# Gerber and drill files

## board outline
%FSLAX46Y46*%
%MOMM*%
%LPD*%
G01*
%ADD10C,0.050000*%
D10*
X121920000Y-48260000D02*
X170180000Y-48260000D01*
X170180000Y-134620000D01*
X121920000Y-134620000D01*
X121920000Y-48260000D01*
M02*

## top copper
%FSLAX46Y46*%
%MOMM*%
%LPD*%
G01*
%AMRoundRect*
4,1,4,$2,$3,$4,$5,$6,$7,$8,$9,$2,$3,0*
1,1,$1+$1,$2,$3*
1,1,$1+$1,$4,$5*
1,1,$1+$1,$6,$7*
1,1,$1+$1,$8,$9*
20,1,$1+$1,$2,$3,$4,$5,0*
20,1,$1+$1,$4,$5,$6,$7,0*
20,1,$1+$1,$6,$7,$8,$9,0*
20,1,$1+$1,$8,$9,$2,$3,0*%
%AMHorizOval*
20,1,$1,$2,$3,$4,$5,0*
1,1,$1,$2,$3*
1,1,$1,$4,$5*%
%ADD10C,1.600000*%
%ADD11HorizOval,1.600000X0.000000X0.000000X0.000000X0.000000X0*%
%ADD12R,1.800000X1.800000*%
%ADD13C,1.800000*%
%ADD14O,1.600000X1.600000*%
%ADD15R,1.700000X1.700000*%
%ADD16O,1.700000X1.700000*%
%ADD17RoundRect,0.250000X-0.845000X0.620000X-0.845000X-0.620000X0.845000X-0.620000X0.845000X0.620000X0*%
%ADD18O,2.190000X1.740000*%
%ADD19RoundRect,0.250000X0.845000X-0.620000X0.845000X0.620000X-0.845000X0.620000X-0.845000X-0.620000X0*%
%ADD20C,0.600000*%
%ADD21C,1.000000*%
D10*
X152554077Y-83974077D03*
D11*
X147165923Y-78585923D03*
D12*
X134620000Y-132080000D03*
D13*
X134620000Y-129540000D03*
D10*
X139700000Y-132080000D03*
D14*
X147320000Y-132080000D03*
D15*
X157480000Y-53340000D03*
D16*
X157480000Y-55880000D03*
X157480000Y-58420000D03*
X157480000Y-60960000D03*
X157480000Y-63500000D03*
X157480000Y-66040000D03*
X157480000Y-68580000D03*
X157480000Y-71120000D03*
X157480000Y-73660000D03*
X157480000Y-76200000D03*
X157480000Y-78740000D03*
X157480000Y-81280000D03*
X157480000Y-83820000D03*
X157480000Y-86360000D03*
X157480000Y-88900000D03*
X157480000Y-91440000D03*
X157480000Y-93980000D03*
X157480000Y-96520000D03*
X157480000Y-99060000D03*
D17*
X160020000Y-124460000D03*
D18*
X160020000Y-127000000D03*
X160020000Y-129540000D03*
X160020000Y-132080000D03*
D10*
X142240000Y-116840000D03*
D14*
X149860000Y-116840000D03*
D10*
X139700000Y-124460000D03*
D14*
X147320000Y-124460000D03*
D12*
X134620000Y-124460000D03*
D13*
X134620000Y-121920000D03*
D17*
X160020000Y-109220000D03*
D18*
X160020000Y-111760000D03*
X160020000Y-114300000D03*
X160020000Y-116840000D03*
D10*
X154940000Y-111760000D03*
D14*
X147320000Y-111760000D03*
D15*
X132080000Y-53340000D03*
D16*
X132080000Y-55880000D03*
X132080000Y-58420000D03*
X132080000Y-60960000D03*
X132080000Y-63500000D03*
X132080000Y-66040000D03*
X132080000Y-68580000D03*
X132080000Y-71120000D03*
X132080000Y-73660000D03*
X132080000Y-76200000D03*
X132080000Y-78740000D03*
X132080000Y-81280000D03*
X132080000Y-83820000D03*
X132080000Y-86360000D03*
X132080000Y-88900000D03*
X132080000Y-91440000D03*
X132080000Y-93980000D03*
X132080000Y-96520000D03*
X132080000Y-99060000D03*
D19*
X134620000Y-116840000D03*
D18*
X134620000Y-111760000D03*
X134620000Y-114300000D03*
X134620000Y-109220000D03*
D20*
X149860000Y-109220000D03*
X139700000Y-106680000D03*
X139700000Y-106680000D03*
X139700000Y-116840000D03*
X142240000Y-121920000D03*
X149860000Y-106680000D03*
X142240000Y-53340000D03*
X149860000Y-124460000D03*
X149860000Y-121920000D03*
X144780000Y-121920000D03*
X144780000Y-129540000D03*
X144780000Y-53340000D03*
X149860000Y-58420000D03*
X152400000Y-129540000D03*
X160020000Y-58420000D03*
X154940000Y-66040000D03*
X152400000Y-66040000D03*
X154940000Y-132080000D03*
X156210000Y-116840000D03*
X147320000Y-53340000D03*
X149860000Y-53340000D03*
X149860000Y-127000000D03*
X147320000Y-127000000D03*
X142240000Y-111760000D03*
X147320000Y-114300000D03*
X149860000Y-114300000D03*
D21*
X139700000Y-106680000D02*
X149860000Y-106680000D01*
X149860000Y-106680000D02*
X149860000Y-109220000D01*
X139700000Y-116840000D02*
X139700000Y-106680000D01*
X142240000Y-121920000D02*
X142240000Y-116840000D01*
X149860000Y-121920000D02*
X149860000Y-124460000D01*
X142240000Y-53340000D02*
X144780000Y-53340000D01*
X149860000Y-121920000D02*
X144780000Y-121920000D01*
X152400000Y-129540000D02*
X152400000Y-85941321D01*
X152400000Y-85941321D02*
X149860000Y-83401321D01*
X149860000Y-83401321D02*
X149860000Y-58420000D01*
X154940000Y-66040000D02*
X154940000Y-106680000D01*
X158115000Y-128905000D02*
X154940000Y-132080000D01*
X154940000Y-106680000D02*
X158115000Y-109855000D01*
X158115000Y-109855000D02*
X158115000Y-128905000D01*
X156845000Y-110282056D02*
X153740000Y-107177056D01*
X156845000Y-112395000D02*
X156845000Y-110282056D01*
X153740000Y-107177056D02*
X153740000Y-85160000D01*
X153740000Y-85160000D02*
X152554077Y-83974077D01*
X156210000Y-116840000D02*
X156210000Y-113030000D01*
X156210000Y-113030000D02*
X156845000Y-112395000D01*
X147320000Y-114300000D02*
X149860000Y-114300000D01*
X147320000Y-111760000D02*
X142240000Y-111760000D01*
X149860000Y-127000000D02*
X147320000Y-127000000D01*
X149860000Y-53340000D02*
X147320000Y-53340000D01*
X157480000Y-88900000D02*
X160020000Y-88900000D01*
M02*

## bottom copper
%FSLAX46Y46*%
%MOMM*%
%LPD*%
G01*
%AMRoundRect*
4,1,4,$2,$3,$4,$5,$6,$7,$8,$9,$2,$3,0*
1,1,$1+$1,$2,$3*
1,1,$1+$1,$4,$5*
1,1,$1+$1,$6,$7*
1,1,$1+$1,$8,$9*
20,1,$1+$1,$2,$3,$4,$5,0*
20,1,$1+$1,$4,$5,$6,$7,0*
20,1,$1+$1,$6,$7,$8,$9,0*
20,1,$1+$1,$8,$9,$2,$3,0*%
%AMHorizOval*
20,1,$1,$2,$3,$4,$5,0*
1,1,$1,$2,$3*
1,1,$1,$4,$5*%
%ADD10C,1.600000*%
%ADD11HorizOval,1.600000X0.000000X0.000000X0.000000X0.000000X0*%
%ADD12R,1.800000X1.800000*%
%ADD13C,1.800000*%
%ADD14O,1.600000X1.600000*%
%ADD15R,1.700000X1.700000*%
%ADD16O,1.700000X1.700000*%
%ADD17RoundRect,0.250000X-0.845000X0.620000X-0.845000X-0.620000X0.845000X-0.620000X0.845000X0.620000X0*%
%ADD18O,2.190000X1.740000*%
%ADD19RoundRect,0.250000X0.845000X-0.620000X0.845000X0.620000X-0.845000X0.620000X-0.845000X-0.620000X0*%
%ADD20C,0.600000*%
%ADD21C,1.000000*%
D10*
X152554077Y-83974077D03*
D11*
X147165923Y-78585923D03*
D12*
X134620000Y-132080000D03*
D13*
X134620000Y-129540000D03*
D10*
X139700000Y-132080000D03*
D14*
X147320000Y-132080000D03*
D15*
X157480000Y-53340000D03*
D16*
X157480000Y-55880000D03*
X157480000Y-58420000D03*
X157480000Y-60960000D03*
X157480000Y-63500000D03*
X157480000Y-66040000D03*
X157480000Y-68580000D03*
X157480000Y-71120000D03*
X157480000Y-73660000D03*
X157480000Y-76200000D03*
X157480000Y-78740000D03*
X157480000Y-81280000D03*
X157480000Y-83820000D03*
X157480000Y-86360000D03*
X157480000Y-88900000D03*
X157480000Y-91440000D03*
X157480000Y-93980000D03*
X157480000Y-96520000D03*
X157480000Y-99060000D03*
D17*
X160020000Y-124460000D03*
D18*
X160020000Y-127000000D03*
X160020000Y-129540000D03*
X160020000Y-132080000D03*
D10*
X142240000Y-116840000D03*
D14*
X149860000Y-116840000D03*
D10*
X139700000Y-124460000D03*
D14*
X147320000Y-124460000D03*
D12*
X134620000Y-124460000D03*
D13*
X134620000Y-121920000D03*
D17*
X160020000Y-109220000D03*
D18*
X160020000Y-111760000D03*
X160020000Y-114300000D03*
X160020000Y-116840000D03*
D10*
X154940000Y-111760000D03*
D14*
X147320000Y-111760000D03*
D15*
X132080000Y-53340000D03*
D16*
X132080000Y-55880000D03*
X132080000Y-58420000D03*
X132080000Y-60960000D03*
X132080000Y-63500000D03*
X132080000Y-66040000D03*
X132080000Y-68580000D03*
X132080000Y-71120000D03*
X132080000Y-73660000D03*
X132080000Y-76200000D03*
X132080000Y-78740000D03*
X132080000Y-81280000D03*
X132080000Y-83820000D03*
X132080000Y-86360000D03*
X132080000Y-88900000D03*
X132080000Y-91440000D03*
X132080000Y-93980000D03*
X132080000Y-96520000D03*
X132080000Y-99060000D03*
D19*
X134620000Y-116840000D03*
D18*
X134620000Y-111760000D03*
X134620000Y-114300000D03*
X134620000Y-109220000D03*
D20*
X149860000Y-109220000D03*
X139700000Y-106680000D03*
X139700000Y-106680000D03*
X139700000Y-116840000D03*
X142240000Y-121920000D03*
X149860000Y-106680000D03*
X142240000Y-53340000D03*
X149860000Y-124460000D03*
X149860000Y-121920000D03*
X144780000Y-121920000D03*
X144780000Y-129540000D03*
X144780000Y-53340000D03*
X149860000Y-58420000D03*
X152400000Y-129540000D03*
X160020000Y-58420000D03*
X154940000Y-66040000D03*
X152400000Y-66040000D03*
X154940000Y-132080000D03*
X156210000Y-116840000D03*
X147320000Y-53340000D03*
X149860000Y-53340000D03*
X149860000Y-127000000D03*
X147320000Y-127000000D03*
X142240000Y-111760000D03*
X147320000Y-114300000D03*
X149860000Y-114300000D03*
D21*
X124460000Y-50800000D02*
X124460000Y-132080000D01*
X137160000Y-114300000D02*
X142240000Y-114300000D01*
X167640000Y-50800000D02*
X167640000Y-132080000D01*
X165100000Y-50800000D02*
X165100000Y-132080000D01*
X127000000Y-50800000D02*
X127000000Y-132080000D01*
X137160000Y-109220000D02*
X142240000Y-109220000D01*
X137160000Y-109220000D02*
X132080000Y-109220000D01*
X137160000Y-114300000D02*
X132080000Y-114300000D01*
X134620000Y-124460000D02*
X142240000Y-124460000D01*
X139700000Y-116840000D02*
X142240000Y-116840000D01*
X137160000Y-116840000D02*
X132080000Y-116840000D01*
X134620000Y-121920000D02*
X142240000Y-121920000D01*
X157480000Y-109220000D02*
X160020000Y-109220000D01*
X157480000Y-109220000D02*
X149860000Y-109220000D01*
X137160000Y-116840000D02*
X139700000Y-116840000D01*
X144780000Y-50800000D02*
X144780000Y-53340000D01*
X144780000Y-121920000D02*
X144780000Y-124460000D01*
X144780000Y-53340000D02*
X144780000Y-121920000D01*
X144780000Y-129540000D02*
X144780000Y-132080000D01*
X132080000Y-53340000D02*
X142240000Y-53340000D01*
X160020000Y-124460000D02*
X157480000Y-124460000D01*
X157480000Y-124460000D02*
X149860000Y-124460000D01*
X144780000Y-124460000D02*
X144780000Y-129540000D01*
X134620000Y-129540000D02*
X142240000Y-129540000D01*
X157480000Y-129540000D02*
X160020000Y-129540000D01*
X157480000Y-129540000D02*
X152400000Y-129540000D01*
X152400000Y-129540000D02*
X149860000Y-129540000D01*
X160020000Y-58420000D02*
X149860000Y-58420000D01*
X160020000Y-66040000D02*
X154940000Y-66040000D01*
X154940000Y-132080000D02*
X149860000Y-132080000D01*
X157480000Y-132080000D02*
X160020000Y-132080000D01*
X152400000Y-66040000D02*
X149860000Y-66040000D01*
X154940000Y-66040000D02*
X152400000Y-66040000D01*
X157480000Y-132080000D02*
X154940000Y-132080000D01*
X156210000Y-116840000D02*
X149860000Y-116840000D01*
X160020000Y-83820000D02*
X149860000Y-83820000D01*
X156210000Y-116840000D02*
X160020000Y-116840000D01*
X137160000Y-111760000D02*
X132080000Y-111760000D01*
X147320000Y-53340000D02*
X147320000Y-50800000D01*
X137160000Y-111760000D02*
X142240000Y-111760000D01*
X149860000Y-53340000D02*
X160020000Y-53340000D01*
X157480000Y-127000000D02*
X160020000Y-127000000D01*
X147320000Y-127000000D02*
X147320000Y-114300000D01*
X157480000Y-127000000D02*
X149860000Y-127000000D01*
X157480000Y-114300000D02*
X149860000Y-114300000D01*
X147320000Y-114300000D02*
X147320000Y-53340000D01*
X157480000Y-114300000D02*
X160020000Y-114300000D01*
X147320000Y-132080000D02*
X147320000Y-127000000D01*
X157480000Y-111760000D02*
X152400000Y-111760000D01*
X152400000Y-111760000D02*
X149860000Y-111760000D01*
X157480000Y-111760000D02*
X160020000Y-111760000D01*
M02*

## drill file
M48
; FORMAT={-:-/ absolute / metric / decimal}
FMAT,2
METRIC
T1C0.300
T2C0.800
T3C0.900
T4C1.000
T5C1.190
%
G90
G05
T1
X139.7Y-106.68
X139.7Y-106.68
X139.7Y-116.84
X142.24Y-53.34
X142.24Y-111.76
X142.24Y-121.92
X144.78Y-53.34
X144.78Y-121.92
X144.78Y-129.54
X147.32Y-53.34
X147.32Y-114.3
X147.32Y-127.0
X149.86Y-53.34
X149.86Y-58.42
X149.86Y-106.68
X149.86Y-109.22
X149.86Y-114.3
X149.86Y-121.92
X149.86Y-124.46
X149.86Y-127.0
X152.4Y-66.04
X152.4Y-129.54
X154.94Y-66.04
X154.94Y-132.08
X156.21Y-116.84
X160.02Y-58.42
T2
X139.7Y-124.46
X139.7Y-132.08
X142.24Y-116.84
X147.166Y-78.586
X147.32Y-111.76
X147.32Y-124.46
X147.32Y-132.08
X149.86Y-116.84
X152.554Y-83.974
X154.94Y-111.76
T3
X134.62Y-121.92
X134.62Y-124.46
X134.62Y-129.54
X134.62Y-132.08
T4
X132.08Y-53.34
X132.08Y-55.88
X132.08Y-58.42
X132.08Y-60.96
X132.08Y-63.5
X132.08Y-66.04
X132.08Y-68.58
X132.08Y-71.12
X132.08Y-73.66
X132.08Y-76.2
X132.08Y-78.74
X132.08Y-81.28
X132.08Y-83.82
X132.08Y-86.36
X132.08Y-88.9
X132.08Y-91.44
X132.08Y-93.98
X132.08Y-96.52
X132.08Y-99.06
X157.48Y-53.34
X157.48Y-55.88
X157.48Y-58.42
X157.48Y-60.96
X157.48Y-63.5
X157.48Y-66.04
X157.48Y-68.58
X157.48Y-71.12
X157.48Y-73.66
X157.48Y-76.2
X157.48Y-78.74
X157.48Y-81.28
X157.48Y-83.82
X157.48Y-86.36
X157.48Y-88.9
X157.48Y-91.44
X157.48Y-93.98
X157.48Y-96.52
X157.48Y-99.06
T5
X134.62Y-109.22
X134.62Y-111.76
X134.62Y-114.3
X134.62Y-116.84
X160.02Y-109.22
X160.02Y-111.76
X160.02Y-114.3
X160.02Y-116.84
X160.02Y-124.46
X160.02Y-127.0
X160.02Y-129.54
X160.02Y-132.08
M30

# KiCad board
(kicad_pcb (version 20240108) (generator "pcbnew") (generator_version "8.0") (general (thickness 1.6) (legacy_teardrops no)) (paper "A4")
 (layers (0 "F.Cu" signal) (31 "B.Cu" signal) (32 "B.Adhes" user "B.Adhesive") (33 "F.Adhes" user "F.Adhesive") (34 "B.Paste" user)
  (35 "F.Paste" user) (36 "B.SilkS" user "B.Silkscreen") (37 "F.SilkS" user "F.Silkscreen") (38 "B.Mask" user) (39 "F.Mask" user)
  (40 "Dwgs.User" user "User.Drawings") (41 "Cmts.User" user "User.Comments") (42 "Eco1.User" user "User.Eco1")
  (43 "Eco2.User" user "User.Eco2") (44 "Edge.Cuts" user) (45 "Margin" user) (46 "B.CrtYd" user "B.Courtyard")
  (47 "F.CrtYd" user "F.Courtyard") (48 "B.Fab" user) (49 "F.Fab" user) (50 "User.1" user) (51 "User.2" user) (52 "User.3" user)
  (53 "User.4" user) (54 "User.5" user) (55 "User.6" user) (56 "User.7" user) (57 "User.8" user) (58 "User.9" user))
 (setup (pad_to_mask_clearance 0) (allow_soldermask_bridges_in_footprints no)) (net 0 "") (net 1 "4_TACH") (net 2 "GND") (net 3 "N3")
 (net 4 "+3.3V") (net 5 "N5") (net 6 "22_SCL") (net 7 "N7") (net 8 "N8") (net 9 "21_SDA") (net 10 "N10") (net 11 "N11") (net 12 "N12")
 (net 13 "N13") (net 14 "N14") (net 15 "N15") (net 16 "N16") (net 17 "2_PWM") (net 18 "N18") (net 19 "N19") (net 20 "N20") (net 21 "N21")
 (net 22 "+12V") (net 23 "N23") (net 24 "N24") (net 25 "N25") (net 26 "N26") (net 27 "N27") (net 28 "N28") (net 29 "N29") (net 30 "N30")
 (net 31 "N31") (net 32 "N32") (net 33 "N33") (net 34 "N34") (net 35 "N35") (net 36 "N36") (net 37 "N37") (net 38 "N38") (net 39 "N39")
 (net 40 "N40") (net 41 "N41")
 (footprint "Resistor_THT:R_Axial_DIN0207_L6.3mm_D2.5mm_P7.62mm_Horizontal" (layer "F.Cu") (at 152.554077 83.974077 135)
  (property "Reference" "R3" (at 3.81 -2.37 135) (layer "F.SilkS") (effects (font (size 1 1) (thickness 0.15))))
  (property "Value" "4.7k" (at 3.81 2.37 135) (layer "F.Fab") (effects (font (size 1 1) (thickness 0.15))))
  (pad "1" thru_hole circle (at 0 0 135) (size 1.6 1.6) (drill 0.8) (layers "*.Cu" "*.Mask") (remove_unused_layers no) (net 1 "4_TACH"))
  (pad "2" thru_hole oval (at 7.62 0 135) (size 1.6 1.6) (drill 0.8) (layers "*.Cu" "*.Mask") (remove_unused_layers no) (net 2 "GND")))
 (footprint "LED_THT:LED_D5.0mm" (layer "F.Cu") (at 134.62 132.08 90)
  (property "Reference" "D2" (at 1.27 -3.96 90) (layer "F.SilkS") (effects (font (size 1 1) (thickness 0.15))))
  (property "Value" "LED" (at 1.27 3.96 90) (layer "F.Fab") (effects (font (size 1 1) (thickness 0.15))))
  (pad "1" thru_hole rect (at 0 0 90) (size 1.8 1.8) (drill 0.9) (layers "*.Cu" "*.Mask") (remove_unused_layers no) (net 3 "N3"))
  (pad "2" thru_hole circle (at 2.54 0 90) (size 1.8 1.8) (drill 0.9) (layers "*.Cu" "*.Mask") (remove_unused_layers no) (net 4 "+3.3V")))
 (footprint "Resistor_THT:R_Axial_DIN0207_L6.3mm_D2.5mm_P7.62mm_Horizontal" (layer "F.Cu") (at 139.7 132.08)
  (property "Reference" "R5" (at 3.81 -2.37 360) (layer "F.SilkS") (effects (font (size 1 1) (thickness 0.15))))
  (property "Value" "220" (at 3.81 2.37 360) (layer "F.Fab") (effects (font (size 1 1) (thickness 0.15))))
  (pad "1" thru_hole circle (at 0 0) (size 1.6 1.6) (drill 0.8) (layers "*.Cu" "*.Mask") (remove_unused_layers no) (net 3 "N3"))
  (pad "2" thru_hole oval (at 7.62 0) (size 1.6 1.6) (drill 0.8) (layers "*.Cu" "*.Mask") (remove_unused_layers no) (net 2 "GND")))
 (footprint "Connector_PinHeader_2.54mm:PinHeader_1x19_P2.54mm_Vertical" (layer "F.Cu") (at 157.48 53.34)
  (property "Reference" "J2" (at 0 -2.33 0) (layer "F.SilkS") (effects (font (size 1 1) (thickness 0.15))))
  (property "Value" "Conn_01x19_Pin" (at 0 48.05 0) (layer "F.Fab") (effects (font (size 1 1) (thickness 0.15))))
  (pad "1" thru_hole rect (at 0 0) (size 1.7 1.7) (drill 1) (layers "*.Cu" "*.Mask") (remove_unused_layers no) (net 2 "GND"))
  (pad "2" thru_hole oval (at 0 2.54) (size 1.7 1.7) (drill 1) (layers "*.Cu" "*.Mask") (remove_unused_layers no) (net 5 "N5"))
  (pad "3" thru_hole oval (at 0 5.08) (size 1.7 1.7) (drill 1) (layers "*.Cu" "*.Mask") (remove_unused_layers no) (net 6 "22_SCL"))
  (pad "4" thru_hole oval (at 0 7.62) (size 1.7 1.7) (drill 1) (layers "*.Cu" "*.Mask") (remove_unused_layers no) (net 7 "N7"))
  (pad "5" thru_hole oval (at 0 10.16) (size 1.7 1.7) (drill 1) (layers "*.Cu" "*.Mask") (remove_unused_layers no) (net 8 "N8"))
  (pad "6" thru_hole oval (at 0 12.7) (size 1.7 1.7) (drill 1) (layers "*.Cu" "*.Mask") (remove_unused_layers no) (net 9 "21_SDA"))
  (pad "7" thru_hole oval (at 0 15.24) (size 1.7 1.7) (drill 1) (layers "*.Cu" "*.Mask") (remove_unused_layers no) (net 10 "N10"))
  (pad "8" thru_hole oval (at 0 17.78) (size 1.7 1.7) (drill 1) (layers "*.Cu" "*.Mask") (remove_unused_layers no) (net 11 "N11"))
  (pad "9" thru_hole oval (at 0 20.32) (size 1.7 1.7) (drill 1) (layers "*.Cu" "*.Mask") (remove_unused_layers no) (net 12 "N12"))
  (pad "10" thru_hole oval (at 0 22.86) (size 1.7 1.7) (drill 1) (layers "*.Cu" "*.Mask") (remove_unused_layers no) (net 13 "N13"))
  (pad "11" thru_hole oval (at 0 25.4) (size 1.7 1.7) (drill 1) (layers "*.Cu" "*.Mask") (remove_unused_layers no) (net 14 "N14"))
  (pad "12" thru_hole oval (at 0 27.94) (size 1.7 1.7) (drill 1) (layers "*.Cu" "*.Mask") (remove_unused_layers no) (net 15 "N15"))
  (pad "13" thru_hole oval (at 0 30.48) (size 1.7 1.7) (drill 1) (layers "*.Cu" "*.Mask") (remove_unused_layers no) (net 1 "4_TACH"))
  (pad "14" thru_hole oval (at 0 33.02) (size 1.7 1.7) (drill 1) (layers "*.Cu" "*.Mask") (remove_unused_layers no) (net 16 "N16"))
  (pad "15" thru_hole oval (at 0 35.56) (size 1.7 1.7) (drill 1) (layers "*.Cu" "*.Mask") (remove_unused_layers no) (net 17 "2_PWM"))
  (pad "16" thru_hole oval (at 0 38.1) (size 1.7 1.7) (drill 1) (layers "*.Cu" "*.Mask") (remove_unused_layers no) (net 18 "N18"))
  (pad "17" thru_hole oval (at 0 40.64) (size 1.7 1.7) (drill 1) (layers "*.Cu" "*.Mask") (remove_unused_layers no) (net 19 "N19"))
  (pad "18" thru_hole oval (at 0 43.18) (size 1.7 1.7) (drill 1) (layers "*.Cu" "*.Mask") (remove_unused_layers no) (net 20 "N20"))
  (pad "19" thru_hole oval (at 0 45.72) (size 1.7 1.7) (drill 1) (layers "*.Cu" "*.Mask") (remove_unused_layers no) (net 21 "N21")))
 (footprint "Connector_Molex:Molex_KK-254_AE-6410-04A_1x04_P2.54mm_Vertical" (layer "F.Cu") (at 160.02 124.46 -90)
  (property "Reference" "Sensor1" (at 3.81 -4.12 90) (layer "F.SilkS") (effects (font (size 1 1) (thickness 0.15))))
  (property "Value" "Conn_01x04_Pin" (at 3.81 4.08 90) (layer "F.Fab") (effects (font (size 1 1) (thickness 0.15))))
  (pad "1" thru_hole roundrect (at 0 0 270) (size 1.74 2.19) (drill 1.19) (layers "*.Cu" "*.Mask") (remove_unused_layers no)
   (roundrect_rratio 0.143678) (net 4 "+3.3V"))
  (pad "2" thru_hole oval (at 2.54 0 270) (size 1.74 2.19) (drill 1.19) (layers "*.Cu" "*.Mask") (remove_unused_layers no) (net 2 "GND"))
  (pad "3" thru_hole oval (at 5.08 0 270) (size 1.74 2.19) (drill 1.19) (layers "*.Cu" "*.Mask") (remove_unused_layers no) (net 6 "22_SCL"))
  (pad "4" thru_hole oval (at 7.62 0 270) (size 1.74 2.19) (drill 1.19) (layers "*.Cu" "*.Mask") (remove_unused_layers no) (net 9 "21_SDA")))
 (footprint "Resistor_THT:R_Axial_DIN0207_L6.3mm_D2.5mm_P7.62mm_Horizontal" (layer "F.Cu") (at 142.24 116.84)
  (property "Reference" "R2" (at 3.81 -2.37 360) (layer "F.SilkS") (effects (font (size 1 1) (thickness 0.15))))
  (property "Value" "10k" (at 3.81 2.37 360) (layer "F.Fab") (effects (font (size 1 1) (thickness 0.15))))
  (pad "1" thru_hole circle (at 0 0) (size 1.6 1.6) (drill 0.8) (layers "*.Cu" "*.Mask") (remove_unused_layers no) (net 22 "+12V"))
  (pad "2" thru_hole oval (at 7.62 0) (size 1.6 1.6) (drill 0.8) (layers "*.Cu" "*.Mask") (remove_unused_layers no) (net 1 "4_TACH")))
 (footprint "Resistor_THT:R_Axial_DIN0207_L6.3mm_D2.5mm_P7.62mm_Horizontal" (layer "F.Cu") (at 139.7 124.46)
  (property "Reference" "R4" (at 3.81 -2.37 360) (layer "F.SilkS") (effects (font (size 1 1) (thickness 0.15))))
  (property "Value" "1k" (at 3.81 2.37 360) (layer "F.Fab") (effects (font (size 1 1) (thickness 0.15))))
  (pad "1" thru_hole circle (at 0 0) (size 1.6 1.6) (drill 0.8) (layers "*.Cu" "*.Mask") (remove_unused_layers no) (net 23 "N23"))
  (pad "2" thru_hole oval (at 7.62 0) (size 1.6 1.6) (drill 0.8) (layers "*.Cu" "*.Mask") (remove_unused_layers no) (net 2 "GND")))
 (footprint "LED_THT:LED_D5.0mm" (layer "F.Cu") (at 134.62 124.46 90)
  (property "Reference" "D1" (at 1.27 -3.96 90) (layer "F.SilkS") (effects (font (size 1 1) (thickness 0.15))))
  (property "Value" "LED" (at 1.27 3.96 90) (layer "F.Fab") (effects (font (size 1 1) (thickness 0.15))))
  (pad "1" thru_hole rect (at 0 0 90) (size 1.8 1.8) (drill 0.9) (layers "*.Cu" "*.Mask") (remove_unused_layers no) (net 23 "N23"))
  (pad "2" thru_hole circle (at 2.54 0 90) (size 1.8 1.8) (drill 0.9) (layers "*.Cu" "*.Mask") (remove_unused_layers no) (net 22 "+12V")))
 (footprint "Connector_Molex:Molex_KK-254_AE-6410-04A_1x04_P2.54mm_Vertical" (layer "F.Cu") (at 160.02 109.22 -90)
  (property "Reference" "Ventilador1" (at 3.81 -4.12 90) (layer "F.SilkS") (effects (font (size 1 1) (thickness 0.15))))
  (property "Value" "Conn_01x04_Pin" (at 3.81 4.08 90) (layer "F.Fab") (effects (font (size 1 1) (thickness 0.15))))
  (pad "1" thru_hole roundrect (at 0 0 270) (size 1.74 2.19) (drill 1.19) (layers "*.Cu" "*.Mask") (remove_unused_layers no)
   (roundrect_rratio 0.143678) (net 22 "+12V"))
  (pad "2" thru_hole oval (at 2.54 0 270) (size 1.74 2.19) (drill 1.19) (layers "*.Cu" "*.Mask") (remove_unused_layers no) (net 17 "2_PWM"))
  (pad "3" thru_hole oval (at 5.08 0 270) (size 1.74 2.19) (drill 1.19) (layers "*.Cu" "*.Mask") (remove_unused_layers no) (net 2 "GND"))
  (pad "4" thru_hole oval (at 7.62 0 270) (size 1.74 2.19) (drill 1.19) (layers "*.Cu" "*.Mask") (remove_unused_layers no) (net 1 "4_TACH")))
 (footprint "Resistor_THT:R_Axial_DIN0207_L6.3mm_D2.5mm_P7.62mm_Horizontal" (layer "F.Cu") (at 154.94 111.76 180)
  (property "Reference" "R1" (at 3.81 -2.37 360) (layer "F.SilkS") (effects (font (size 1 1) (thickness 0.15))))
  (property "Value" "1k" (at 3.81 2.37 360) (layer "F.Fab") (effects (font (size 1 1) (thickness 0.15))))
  (pad "1" thru_hole circle (at 0 0 180) (size 1.6 1.6) (drill 0.8) (layers "*.Cu" "*.Mask") (remove_unused_layers no) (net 17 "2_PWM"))
  (pad "2" thru_hole oval (at 7.62 0 180) (size 1.6 1.6) (drill 0.8) (layers "*.Cu" "*.Mask") (remove_unused_layers no) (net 2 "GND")))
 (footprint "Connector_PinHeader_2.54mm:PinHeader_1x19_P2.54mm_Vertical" (layer "F.Cu") (at 132.08 53.34)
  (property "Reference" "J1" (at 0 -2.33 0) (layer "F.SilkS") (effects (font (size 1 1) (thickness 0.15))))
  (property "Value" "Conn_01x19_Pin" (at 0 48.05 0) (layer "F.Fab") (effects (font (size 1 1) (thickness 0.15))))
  (pad "1" thru_hole rect (at 0 0) (size 1.7 1.7) (drill 1) (layers "*.Cu" "*.Mask") (remove_unused_layers no) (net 4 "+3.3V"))
  (pad "2" thru_hole oval (at 0 2.54) (size 1.7 1.7) (drill 1) (layers "*.Cu" "*.Mask") (remove_unused_layers no) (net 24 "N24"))
  (pad "3" thru_hole oval (at 0 5.08) (size 1.7 1.7) (drill 1) (layers "*.Cu" "*.Mask") (remove_unused_layers no) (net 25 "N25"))
  (pad "4" thru_hole oval (at 0 7.62) (size 1.7 1.7) (drill 1) (layers "*.Cu" "*.Mask") (remove_unused_layers no) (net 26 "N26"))
  (pad "5" thru_hole oval (at 0 10.16) (size 1.7 1.7) (drill 1) (layers "*.Cu" "*.Mask") (remove_unused_layers no) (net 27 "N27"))
  (pad "6" thru_hole oval (at 0 12.7) (size 1.7 1.7) (drill 1) (layers "*.Cu" "*.Mask") (remove_unused_layers no) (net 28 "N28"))
  (pad "7" thru_hole oval (at 0 15.24) (size 1.7 1.7) (drill 1) (layers "*.Cu" "*.Mask") (remove_unused_layers no) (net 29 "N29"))
  (pad "8" thru_hole oval (at 0 17.78) (size 1.7 1.7) (drill 1) (layers "*.Cu" "*.Mask") (remove_unused_layers no) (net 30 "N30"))
  (pad "9" thru_hole oval (at 0 20.32) (size 1.7 1.7) (drill 1) (layers "*.Cu" "*.Mask") (remove_unused_layers no) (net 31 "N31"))
  (pad "10" thru_hole oval (at 0 22.86) (size 1.7 1.7) (drill 1) (layers "*.Cu" "*.Mask") (remove_unused_layers no) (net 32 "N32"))
  (pad "11" thru_hole oval (at 0 25.4) (size 1.7 1.7) (drill 1) (layers "*.Cu" "*.Mask") (remove_unused_layers no) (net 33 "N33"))
  (pad "12" thru_hole oval (at 0 27.94) (size 1.7 1.7) (drill 1) (layers "*.Cu" "*.Mask") (remove_unused_layers no) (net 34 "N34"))
  (pad "13" thru_hole oval (at 0 30.48) (size 1.7 1.7) (drill 1) (layers "*.Cu" "*.Mask") (remove_unused_layers no) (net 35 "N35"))
  (pad "14" thru_hole oval (at 0 33.02) (size 1.7 1.7) (drill 1) (layers "*.Cu" "*.Mask") (remove_unused_layers no) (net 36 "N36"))
  (pad "15" thru_hole oval (at 0 35.56) (size 1.7 1.7) (drill 1) (layers "*.Cu" "*.Mask") (remove_unused_layers no) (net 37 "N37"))
  (pad "16" thru_hole oval (at 0 38.1) (size 1.7 1.7) (drill 1) (layers "*.Cu" "*.Mask") (remove_unused_layers no) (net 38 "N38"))
  (pad "17" thru_hole oval (at 0 40.64) (size 1.7 1.7) (drill 1) (layers "*.Cu" "*.Mask") (remove_unused_layers no) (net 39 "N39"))
  (pad "18" thru_hole oval (at 0 43.18) (size 1.7 1.7) (drill 1) (layers "*.Cu" "*.Mask") (remove_unused_layers no) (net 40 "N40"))
  (pad "19" thru_hole oval (at 0 45.72) (size 1.7 1.7) (drill 1) (layers "*.Cu" "*.Mask") (remove_unused_layers no) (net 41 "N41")))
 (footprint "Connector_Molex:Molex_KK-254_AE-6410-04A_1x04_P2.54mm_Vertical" (layer "F.Cu") (at 134.62 116.84 90)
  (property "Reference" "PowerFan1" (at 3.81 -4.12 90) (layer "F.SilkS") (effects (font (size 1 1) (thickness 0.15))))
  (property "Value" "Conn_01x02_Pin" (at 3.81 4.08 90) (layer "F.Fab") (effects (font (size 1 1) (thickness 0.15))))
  (pad "1" thru_hole roundrect (at 0 0 90) (size 1.74 2.19) (drill 1.19) (layers "*.Cu" "*.Mask") (remove_unused_layers no)
   (roundrect_rratio 0.143678) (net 22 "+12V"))
  (pad "2" thru_hole oval (at 5.08 0 90) (size 1.74 2.19) (drill 1.19) (layers "*.Cu" "*.Mask") (remove_unused_layers no) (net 2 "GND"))
  (pad "3" thru_hole oval (at 2.54 0 90) (size 1.74 2.19) (drill 1.19) (layers "*.Cu" "*.Mask") (remove_unused_layers no))
  (pad "4" thru_hole oval (at 7.62 0 90) (size 1.74 2.19) (drill 1.19) (layers "*.Cu" "*.Mask") (remove_unused_layers no)))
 (gr_rect (start 121.92 48.26) (end 170.18 134.62) (stroke (width 0.05) (type default)) (fill none) (layer "Edge.Cuts"))
 (segment (start 124.46 50.8) (end 124.46 132.08) (width 1) (layer "B.Cu") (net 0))
 (segment (start 137.16 114.3) (end 142.24 114.3) (width 1) (layer "B.Cu") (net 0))
 (segment (start 167.64 50.8) (end 167.64 132.08) (width 1) (layer "B.Cu") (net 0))
 (segment (start 165.1 50.8) (end 165.1 132.08) (width 1) (layer "B.Cu") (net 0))
 (segment (start 127 50.8) (end 127 132.08) (width 1) (layer "B.Cu") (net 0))
 (segment (start 137.16 109.22) (end 142.24 109.22) (width 1) (layer "B.Cu") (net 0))
 (segment (start 137.16 109.22) (end 132.08 109.22) (width 1) (layer "B.Cu") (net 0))
 (segment (start 137.16 114.3) (end 132.08 114.3) (width 1) (layer "B.Cu") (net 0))
 (segment (start 134.62 124.46) (end 142.24 124.46) (width 1) (layer "B.Cu") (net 23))
 (segment (start 139.7 106.68) (end 149.86 106.68) (width 1) (layer "F.Cu") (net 22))
 (segment (start 149.86 106.68) (end 149.86 109.22) (width 1) (layer "F.Cu") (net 22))
 (segment (start 139.7 116.84) (end 139.7 106.68) (width 1) (layer "F.Cu") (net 22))
 (segment (start 142.24 121.92) (end 142.24 116.84) (width 1) (layer "F.Cu") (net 22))
 (via (at 149.86 109.22) (size 0.6) (drill 0.3) (layers "F.Cu" "B.Cu") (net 22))
 (via (at 139.7 106.68) (size 0.6) (drill 0.3) (layers "F.Cu" "B.Cu") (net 22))
 (via (at 139.7 106.68) (size 0.6) (drill 0.3) (layers "F.Cu" "B.Cu") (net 22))
 (via (at 139.7 116.84) (size 0.6) (drill 0.3) (layers "F.Cu" "B.Cu") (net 22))
 (via (at 142.24 121.92) (size 0.6) (drill 0.3) (layers "F.Cu" "B.Cu") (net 22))
 (via (at 149.86 106.68) (size 0.6) (drill 0.3) (layers "F.Cu" "B.Cu") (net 22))
 (segment (start 139.7 116.84) (end 142.24 116.84) (width 1) (layer "B.Cu") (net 22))
 (segment (start 137.16 116.84) (end 132.08 116.84) (width 1) (layer "B.Cu") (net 22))
 (segment (start 134.62 121.92) (end 142.24 121.92) (width 1) (layer "B.Cu") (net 22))
 (segment (start 157.48 109.22) (end 160.02 109.22) (width 1) (layer "B.Cu") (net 22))
 (segment (start 157.48 109.22) (end 149.86 109.22) (width 1) (layer "B.Cu") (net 22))
 (segment (start 137.16 116.84) (end 139.7 116.84) (width 1) (layer "B.Cu") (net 22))
 (segment (start 149.86 121.92) (end 149.86 124.46) (width 1) (layer "F.Cu") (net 4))
 (segment (start 142.24 53.34) (end 144.78 53.34) (width 1) (layer "F.Cu") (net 4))
 (segment (start 149.86 121.92) (end 144.78 121.92) (width 1) (layer "F.Cu") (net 4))
 (via (at 142.24 53.34) (size 0.6) (drill 0.3) (layers "F.Cu" "B.Cu") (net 4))
 (via (at 149.86 124.46) (size 0.6) (drill 0.3) (layers "F.Cu" "B.Cu") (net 4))
 (via (at 149.86 121.92) (size 0.6) (drill 0.3) (layers "F.Cu" "B.Cu") (free yes) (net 4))
 (via (at 144.78 121.92) (size 0.6) (drill 0.3) (layers "F.Cu" "B.Cu") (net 4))
 (via (at 144.78 129.54) (size 0.6) (drill 0.3) (layers "F.Cu" "B.Cu") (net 4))
 (via (at 144.78 53.34) (size 0.6) (drill 0.3) (layers "F.Cu" "B.Cu") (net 4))
 (segment (start 144.78 50.8) (end 144.78 53.34) (width 1) (layer "B.Cu") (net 4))
 (segment (start 144.78 121.92) (end 144.78 124.46) (width 1) (layer "B.Cu") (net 4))
 (segment (start 144.78 53.34) (end 144.78 121.92) (width 1) (layer "B.Cu") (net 4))
 (segment (start 144.78 129.54) (end 144.78 132.08) (width 1) (layer "B.Cu") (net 4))
 (segment (start 132.08 53.34) (end 142.24 53.34) (width 1) (layer "B.Cu") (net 4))
 (segment (start 160.02 124.46) (end 157.48 124.46) (width 1) (layer "B.Cu") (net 4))
 (segment (start 157.48 124.46) (end 149.86 124.46) (width 1) (layer "B.Cu") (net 4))
 (segment (start 144.78 124.46) (end 144.78 129.54) (width 1) (layer "B.Cu") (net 4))
 (segment (start 134.62 129.54) (end 142.24 129.54) (width 1) (layer "B.Cu") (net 4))
 (segment (start 152.4 129.54) (end 152.4 85.941321) (width 1) (layer "F.Cu") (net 6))
 (segment (start 152.4 85.941321) (end 149.86 83.401321) (width 1) (layer "F.Cu") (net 6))
 (segment (start 149.86 83.401321) (end 149.86 58.42) (width 1) (layer "F.Cu") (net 6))
 (via (at 149.86 58.42) (size 0.6) (drill 0.3) (layers "F.Cu" "B.Cu") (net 6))
 (via (at 152.4 129.54) (size 0.6) (drill 0.3) (layers "F.Cu" "B.Cu") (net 6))
 (via (at 160.02 58.42) (size 0.6) (drill 0.3) (layers "F.Cu" "B.Cu") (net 6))
 (segment (start 157.48 129.54) (end 160.02 129.54) (width 1) (layer "B.Cu") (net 6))
 (segment (start 157.48 129.54) (end 152.4 129.54) (width 1) (layer "B.Cu") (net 6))
 (segment (start 152.4 129.54) (end 149.86 129.54) (width 1) (layer "B.Cu") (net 6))
 (segment (start 160.02 58.42) (end 149.86 58.42) (width 1) (layer "B.Cu") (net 6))
 (segment (start 154.94 66.04) (end 154.94 106.68) (width 1) (layer "F.Cu") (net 9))
 (segment (start 158.115 128.905) (end 154.94 132.08) (width 1) (layer "F.Cu") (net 9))
 (segment (start 154.94 106.68) (end 158.115 109.855) (width 1) (layer "F.Cu") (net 9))
 (segment (start 158.115 109.855) (end 158.115 128.905) (width 1) (layer "F.Cu") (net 9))
 (via (at 154.94 66.04) (size 0.6) (drill 0.3) (layers "F.Cu" "B.Cu") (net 9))
 (via (at 152.4 66.04) (size 0.6) (drill 0.3) (layers "F.Cu" "B.Cu") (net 9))
 (via (at 154.94 132.08) (size 0.6) (drill 0.3) (layers "F.Cu" "B.Cu") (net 9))
 (segment (start 160.02 66.04) (end 154.94 66.04) (width 1) (layer "B.Cu") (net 9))
 (segment (start 154.94 132.08) (end 149.86 132.08) (width 1) (layer "B.Cu") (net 9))
 (segment (start 157.48 132.08) (end 160.02 132.08) (width 1) (layer "B.Cu") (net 9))
 (segment (start 152.4 66.04) (end 149.86 66.04) (width 1) (layer "B.Cu") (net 9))
 (segment (start 154.94 66.04) (end 152.4 66.04) (width 1) (layer "B.Cu") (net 9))
 (segment (start 157.48 132.08) (end 154.94 132.08) (width 1) (layer "B.Cu") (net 9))
 (segment (start 156.845 110.282056) (end 153.74 107.177056) (width 1) (layer "F.Cu") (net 1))
 (segment (start 156.845 112.395) (end 156.845 110.282056) (width 1) (layer "F.Cu") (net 1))
 (segment (start 153.74 107.177056) (end 153.74 85.16) (width 1) (layer "F.Cu") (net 1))
 (segment (start 153.74 85.16) (end 152.554077 83.974077) (width 1) (layer "F.Cu") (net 1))
 (segment (start 156.21 116.84) (end 156.21 113.03) (width 1) (layer "F.Cu") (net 1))
 (segment (start 156.21 113.03) (end 156.845 112.395) (width 1) (layer "F.Cu") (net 1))
 (via (at 156.21 116.84) (size 0.6) (drill 0.3) (layers "F.Cu" "B.Cu") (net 1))
 (segment (start 156.21 116.84) (end 149.86 116.84) (width 1) (layer "B.Cu") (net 1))
 (segment (start 160.02 83.82) (end 149.86 83.82) (width 1) (layer "B.Cu") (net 1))
 (segment (start 156.21 116.84) (end 160.02 116.84) (width 1) (layer "B.Cu") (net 1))
 (segment (start 147.32 114.3) (end 149.86 114.3) (width 1) (layer "F.Cu") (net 2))
 (segment (start 147.32 111.76) (end 142.24 111.76) (width 1) (layer "F.Cu") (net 2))
 (segment (start 149.86 127) (end 147.32 127) (width 1) (layer "F.Cu") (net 2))
 (segment (start 149.86 53.34) (end 147.32 53.34) (width 1) (layer "F.Cu") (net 2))
 (via (at 147.32 53.34) (size 0.6) (drill 0.3) (layers "F.Cu" "B.Cu") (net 2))
 (via (at 149.86 53.34) (size 0.6) (drill 0.3) (layers "F.Cu" "B.Cu") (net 2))
 (via (at 149.86 127) (size 0.6) (drill 0.3) (layers "F.Cu" "B.Cu") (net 2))
 (via (at 147.32 127) (size 0.6) (drill 0.3) (layers "F.Cu" "B.Cu") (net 2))
 (via (at 142.24 111.76) (size 0.6) (drill 0.3) (layers "F.Cu" "B.Cu") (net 2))
 (via (at 147.32 114.3) (size 0.6) (drill 0.3) (layers "F.Cu" "B.Cu") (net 2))
 (via (at 149.86 114.3) (size 0.6) (drill 0.3) (layers "F.Cu" "B.Cu") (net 2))
 (segment (start 137.16 111.76) (end 132.08 111.76) (width 1) (layer "B.Cu") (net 2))
 (segment (start 147.32 53.34) (end 147.32 50.8) (width 1) (layer "B.Cu") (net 2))
 (segment (start 137.16 111.76) (end 142.24 111.76) (width 1) (layer "B.Cu") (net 2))
 (segment (start 149.86 53.34) (end 160.02 53.34) (width 1) (layer "B.Cu") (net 2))
 (segment (start 157.48 127) (end 160.02 127) (width 1) (layer "B.Cu") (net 2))
 (segment (start 147.32 127) (end 147.32 114.3) (width 1) (layer "B.Cu") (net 2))
 (segment (start 157.48 127) (end 149.86 127) (width 1) (layer "B.Cu") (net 2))
 (segment (start 157.48 114.3) (end 149.86 114.3) (width 1) (layer "B.Cu") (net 2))
 (segment (start 147.32 114.3) (end 147.32 53.34) (width 1) (layer "B.Cu") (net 2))
 (segment (start 157.48 114.3) (end 160.02 114.3) (width 1) (layer "B.Cu") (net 2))
 (segment (start 147.32 132.08) (end 147.32 127) (width 1) (layer "B.Cu") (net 2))
 (segment (start 157.48 88.9) (end 160.02 88.9) (width 1) (layer "F.Cu") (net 17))
 (segment (start 157.48 111.76) (end 152.4 111.76) (width 1) (layer "B.Cu") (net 17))
 (segment (start 152.4 111.76) (end 149.86 111.76) (width 1) (layer "B.Cu") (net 17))
 (segment (start 157.48 111.76) (end 160.02 111.76) (width 1) (layer "B.Cu") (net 17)))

